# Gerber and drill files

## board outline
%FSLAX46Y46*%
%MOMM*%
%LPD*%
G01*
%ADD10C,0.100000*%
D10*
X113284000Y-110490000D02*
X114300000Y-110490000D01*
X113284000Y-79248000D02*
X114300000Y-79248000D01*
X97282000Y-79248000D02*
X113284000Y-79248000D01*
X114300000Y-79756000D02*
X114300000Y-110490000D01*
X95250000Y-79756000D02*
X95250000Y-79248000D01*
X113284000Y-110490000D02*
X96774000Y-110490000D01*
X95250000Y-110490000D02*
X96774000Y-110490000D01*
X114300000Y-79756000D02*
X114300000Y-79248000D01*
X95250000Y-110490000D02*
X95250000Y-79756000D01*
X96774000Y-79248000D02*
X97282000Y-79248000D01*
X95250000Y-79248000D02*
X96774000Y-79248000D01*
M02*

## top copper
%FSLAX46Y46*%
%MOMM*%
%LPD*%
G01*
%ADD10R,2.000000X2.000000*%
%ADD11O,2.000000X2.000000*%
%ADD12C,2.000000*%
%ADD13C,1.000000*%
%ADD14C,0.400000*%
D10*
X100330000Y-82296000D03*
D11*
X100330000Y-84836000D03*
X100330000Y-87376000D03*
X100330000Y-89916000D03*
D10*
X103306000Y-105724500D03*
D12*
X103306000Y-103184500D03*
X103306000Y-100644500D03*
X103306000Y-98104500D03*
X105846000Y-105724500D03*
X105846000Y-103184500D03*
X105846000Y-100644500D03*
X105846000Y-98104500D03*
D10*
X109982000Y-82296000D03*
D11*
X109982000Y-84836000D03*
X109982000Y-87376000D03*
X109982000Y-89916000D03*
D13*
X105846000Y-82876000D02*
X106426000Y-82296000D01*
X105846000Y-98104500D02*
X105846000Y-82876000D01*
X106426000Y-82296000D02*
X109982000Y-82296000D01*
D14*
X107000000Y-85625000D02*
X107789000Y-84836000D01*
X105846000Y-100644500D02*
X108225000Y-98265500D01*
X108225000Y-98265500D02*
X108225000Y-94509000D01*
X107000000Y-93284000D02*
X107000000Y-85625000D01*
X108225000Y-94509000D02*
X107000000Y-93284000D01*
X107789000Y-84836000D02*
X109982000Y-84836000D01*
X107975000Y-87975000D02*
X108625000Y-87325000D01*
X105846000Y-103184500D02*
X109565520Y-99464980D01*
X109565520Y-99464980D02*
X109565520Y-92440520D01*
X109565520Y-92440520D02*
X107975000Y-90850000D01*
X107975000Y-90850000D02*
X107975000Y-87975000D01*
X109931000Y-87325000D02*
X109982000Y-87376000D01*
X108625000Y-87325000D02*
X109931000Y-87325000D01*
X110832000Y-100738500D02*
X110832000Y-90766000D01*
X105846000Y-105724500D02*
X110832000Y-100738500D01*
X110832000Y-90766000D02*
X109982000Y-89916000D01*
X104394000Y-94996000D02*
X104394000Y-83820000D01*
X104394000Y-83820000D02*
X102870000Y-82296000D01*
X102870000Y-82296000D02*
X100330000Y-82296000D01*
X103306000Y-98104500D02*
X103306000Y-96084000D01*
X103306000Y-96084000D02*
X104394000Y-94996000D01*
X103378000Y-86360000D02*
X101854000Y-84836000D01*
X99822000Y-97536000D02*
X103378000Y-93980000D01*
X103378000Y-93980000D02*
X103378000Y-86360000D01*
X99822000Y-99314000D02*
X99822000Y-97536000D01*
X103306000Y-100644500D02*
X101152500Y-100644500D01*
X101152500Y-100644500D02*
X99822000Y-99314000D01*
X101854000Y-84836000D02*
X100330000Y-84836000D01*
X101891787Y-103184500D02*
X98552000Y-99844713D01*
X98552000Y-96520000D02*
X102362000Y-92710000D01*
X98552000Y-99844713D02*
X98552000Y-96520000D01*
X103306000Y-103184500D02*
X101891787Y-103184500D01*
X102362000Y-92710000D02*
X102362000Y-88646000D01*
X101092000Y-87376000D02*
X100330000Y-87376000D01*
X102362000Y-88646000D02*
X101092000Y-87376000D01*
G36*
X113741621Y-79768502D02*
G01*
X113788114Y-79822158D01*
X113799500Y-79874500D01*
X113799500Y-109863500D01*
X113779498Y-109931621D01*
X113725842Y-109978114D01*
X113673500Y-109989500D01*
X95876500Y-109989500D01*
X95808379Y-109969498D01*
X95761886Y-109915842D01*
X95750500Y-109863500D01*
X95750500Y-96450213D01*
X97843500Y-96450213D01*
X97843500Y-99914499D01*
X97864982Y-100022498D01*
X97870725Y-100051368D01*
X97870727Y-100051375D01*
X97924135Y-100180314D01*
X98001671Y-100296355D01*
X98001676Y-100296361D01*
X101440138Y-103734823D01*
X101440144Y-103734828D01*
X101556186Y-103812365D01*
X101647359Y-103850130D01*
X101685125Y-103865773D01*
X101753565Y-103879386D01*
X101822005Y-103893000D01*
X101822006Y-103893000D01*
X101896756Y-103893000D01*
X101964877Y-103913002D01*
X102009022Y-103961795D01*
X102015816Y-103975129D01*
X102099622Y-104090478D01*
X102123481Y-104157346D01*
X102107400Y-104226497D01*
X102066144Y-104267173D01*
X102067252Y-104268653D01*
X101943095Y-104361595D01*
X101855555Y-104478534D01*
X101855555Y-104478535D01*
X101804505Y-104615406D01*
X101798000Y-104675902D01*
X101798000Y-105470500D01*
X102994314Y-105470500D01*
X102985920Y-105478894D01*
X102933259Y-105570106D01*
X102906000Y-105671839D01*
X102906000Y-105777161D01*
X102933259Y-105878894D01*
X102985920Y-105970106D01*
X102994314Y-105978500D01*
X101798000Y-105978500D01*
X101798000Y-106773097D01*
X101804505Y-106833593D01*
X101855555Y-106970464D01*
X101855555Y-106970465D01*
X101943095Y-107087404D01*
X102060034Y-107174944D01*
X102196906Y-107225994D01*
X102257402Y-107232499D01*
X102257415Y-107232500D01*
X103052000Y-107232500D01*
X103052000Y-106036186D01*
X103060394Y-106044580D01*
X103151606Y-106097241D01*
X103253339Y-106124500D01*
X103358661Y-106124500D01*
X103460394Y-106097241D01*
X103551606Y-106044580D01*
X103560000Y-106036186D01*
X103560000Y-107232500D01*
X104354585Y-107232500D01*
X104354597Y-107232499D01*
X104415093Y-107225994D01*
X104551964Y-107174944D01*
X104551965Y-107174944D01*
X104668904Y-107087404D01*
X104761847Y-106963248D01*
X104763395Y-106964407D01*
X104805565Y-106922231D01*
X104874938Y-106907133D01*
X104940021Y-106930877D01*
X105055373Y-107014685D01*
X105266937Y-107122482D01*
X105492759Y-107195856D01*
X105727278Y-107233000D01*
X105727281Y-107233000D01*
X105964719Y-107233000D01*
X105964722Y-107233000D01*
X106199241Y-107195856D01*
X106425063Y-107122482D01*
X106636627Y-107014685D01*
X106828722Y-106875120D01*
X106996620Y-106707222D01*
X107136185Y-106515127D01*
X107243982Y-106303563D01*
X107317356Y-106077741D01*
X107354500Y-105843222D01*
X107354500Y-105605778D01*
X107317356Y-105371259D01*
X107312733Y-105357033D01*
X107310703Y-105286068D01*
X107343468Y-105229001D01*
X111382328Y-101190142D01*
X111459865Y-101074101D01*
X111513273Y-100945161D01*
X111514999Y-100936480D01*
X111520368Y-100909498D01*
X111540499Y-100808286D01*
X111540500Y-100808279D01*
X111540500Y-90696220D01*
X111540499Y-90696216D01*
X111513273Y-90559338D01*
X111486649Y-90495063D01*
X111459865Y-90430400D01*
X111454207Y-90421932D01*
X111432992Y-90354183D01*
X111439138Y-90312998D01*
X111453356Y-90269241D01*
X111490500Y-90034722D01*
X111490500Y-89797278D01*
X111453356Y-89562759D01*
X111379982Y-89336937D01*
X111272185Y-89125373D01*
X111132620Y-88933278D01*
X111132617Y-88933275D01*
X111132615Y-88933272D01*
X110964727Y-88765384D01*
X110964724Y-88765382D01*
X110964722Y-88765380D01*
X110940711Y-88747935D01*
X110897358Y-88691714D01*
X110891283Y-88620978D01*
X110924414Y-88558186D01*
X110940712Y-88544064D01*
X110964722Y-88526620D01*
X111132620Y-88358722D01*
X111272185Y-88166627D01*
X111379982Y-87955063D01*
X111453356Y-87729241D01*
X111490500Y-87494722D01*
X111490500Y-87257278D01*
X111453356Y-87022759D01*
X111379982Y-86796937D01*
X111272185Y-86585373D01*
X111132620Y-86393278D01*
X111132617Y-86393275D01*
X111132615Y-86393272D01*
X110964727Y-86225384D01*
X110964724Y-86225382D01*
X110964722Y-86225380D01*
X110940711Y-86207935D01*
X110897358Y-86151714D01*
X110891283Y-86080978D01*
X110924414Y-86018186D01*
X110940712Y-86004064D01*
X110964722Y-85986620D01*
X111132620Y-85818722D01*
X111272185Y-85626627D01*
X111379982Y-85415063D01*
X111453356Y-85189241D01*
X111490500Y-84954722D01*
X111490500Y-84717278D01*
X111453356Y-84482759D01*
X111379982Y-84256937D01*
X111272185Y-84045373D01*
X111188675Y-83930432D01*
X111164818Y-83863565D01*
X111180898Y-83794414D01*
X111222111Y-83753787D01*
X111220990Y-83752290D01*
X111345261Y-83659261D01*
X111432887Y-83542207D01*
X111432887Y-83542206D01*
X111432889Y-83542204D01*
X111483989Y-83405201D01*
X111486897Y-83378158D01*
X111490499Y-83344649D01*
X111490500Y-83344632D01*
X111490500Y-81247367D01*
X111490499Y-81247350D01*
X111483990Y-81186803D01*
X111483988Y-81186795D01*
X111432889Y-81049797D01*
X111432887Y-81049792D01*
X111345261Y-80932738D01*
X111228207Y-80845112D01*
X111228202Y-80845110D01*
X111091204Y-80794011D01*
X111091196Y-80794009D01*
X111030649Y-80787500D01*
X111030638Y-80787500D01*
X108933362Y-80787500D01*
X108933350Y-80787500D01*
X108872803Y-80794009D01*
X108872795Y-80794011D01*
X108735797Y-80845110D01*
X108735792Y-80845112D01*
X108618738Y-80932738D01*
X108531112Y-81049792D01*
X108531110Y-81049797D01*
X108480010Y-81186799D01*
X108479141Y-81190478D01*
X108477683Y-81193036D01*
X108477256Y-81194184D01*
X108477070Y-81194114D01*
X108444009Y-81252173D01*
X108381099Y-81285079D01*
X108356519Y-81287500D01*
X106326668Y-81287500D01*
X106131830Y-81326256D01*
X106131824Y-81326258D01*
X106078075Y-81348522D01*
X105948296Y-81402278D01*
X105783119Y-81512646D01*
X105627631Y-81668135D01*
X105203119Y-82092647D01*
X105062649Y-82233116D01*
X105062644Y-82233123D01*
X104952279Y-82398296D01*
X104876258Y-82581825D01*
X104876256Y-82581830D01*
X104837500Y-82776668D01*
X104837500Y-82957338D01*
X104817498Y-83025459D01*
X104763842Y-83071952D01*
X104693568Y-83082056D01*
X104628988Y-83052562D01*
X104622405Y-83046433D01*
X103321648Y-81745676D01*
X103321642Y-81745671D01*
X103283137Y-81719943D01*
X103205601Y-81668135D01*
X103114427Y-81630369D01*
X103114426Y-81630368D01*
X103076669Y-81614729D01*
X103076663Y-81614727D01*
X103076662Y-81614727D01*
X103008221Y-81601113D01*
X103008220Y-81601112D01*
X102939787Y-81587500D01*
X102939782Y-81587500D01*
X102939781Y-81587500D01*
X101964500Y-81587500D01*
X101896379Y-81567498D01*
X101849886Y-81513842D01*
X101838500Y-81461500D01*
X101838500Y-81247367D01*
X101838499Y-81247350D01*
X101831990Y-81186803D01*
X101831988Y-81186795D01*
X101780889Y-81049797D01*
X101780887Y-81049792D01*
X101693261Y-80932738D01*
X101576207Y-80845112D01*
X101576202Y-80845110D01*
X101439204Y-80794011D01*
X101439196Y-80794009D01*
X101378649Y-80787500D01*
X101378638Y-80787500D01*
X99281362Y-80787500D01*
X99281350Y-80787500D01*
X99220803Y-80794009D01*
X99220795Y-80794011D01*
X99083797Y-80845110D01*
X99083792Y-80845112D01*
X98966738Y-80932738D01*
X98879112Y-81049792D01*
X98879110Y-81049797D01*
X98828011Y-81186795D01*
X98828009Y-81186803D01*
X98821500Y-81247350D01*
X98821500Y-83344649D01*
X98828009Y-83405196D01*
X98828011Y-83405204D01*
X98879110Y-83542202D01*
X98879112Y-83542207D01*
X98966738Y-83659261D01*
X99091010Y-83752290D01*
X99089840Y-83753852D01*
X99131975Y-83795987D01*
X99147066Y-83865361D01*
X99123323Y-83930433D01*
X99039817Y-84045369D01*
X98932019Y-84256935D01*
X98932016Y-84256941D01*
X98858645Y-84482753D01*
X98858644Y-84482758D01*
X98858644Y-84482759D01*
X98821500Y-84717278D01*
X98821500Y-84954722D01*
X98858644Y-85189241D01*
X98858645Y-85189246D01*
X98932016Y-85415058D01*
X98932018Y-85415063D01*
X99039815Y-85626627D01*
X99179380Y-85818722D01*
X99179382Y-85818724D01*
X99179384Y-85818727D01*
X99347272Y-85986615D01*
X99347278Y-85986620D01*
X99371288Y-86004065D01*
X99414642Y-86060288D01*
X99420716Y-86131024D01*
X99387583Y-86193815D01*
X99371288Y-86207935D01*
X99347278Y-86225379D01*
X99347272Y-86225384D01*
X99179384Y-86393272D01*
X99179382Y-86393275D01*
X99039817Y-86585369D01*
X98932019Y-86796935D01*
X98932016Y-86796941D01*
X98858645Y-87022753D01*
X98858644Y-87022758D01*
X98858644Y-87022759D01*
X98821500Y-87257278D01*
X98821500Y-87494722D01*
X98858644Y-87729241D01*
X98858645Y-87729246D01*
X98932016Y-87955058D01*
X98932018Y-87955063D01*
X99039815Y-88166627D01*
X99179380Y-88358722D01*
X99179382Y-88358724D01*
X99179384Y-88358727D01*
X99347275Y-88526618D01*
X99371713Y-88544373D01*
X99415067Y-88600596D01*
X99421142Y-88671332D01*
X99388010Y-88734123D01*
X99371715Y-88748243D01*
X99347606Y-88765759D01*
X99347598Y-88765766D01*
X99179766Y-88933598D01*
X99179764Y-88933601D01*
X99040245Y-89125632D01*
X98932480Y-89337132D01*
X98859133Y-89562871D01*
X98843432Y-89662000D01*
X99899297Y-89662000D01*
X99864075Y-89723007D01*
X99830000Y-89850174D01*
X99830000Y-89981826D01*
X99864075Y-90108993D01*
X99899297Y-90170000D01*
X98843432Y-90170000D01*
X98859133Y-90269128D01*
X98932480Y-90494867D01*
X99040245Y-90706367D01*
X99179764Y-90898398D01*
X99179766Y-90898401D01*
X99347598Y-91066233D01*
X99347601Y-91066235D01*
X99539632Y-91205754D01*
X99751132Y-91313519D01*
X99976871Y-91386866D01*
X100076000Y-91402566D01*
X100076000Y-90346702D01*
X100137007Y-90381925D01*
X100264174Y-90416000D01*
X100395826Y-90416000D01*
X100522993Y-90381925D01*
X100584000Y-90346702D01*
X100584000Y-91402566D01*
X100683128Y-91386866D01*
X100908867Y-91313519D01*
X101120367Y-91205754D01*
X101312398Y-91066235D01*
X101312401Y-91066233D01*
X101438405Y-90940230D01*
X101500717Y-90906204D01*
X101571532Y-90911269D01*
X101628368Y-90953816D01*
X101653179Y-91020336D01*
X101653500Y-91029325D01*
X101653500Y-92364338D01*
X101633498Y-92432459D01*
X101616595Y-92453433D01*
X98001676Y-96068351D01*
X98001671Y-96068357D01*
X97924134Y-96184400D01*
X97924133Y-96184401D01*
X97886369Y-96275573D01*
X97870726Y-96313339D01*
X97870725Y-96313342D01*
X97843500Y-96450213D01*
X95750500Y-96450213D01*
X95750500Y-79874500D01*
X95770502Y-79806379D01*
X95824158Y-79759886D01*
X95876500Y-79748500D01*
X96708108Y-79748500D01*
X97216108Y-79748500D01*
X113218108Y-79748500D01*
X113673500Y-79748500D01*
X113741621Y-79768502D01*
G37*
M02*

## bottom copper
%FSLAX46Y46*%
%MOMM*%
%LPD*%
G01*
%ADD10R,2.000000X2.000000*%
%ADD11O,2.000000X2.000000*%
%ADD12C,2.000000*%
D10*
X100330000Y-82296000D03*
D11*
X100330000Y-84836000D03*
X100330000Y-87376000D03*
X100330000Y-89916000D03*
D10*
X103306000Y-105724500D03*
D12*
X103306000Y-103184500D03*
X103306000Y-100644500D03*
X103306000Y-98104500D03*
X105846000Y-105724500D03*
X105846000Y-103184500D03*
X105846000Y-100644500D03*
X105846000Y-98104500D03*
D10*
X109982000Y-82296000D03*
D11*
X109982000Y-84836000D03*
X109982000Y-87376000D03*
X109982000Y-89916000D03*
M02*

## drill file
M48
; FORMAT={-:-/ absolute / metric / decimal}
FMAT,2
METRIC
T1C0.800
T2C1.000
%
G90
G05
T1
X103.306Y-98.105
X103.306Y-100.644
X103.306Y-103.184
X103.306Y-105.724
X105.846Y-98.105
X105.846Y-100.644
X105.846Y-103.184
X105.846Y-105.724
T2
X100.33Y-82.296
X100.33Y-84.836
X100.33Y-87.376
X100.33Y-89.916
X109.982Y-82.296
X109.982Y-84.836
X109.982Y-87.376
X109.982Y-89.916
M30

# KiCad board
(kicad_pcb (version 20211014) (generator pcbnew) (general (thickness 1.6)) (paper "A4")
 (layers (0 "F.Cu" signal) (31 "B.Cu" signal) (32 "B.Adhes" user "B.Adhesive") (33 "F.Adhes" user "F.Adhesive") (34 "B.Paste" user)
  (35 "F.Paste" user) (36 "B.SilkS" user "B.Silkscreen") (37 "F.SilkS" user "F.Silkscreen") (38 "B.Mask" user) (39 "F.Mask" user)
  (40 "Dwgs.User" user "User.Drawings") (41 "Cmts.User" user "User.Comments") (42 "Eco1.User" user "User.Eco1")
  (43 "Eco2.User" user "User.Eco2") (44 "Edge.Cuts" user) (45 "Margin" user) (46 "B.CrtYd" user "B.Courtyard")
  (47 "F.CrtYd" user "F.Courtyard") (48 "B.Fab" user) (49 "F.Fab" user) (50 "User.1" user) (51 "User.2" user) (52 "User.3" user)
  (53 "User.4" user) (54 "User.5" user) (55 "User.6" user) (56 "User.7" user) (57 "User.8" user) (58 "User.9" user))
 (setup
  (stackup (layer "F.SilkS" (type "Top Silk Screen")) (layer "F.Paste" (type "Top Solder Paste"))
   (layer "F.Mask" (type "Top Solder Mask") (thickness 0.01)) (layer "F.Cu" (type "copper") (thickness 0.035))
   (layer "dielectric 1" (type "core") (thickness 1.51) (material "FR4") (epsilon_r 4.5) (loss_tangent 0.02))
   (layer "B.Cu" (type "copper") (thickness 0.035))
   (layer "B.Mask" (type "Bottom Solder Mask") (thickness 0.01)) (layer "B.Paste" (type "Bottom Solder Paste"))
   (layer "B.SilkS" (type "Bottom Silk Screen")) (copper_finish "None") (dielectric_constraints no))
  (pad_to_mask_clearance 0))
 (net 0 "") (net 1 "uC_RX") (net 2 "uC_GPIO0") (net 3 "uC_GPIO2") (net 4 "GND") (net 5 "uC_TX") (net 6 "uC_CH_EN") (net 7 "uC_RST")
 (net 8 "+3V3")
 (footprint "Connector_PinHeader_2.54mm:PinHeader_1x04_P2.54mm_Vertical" (layer "F.Cu") (at 100.33 82.296)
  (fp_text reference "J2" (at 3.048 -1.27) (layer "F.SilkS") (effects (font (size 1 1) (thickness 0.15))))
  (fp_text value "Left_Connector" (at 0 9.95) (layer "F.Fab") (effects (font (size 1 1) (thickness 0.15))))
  (pad "1" thru_hole rect (at 0 0) (size 2 2) (drill 1) (layers *.Cu *.Mask) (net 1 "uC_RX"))
  (pad "2" thru_hole oval (at 0 2.54) (size 2 2) (drill 1) (layers *.Cu *.Mask) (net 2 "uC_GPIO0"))
  (pad "3" thru_hole oval (at 0 5.08) (size 2 2) (drill 1) (layers *.Cu *.Mask) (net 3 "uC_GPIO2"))
  (pad "4" thru_hole oval (at 0 7.62) (size 2 2) (drill 1) (layers *.Cu *.Mask) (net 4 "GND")))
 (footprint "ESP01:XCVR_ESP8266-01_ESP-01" (layer "F.Cu") (at 94.996 101.9145 90)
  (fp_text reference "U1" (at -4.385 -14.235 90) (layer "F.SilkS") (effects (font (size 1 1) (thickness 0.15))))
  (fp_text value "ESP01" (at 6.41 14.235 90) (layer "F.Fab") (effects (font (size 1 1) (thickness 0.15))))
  (pad "1" thru_hole rect (at -3.81 8.31 90) (size 2 2) (drill 0.8) (layers *.Cu *.Mask) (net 4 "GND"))
  (pad "2" thru_hole circle (at -1.27 8.31 90) (size 2 2) (drill 0.8) (layers *.Cu *.Mask) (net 3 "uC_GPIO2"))
  (pad "3" thru_hole circle (at 1.27 8.31 90) (size 2 2) (drill 0.8) (layers *.Cu *.Mask) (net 2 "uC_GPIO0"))
  (pad "4" thru_hole circle (at 3.81 8.31 90) (size 2 2) (drill 0.8) (layers *.Cu *.Mask) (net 1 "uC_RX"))
  (pad "5" thru_hole circle (at -3.81 10.85 90) (size 2 2) (drill 0.8) (layers *.Cu *.Mask) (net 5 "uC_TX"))
  (pad "6" thru_hole circle (at -1.27 10.85 90) (size 2 2) (drill 0.8) (layers *.Cu *.Mask) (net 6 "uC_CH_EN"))
  (pad "7" thru_hole circle (at 1.27 10.85 90) (size 2 2) (drill 0.8) (layers *.Cu *.Mask) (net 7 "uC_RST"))
  (pad "8" thru_hole circle (at 3.81 10.85 90) (size 2 2) (drill 0.8) (layers *.Cu *.Mask) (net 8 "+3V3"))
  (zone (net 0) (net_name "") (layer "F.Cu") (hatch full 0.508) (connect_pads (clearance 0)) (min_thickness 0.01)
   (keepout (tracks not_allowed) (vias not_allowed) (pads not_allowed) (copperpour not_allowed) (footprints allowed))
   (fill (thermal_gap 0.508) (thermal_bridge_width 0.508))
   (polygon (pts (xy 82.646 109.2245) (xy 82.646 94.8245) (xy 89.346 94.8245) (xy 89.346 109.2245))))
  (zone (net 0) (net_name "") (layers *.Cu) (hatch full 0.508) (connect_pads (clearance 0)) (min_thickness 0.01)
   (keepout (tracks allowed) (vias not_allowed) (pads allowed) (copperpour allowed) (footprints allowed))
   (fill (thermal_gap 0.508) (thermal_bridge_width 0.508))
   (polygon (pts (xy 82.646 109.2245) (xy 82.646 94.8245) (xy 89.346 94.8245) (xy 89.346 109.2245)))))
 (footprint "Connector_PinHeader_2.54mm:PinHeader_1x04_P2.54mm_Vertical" (layer "F.Cu") (at 109.982 82.296)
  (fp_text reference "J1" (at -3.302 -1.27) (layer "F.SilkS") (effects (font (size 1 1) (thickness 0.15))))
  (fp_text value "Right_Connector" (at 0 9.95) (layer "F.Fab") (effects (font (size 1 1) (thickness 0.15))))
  (pad "1" thru_hole rect (at 0 0) (size 2 2) (drill 1) (layers *.Cu *.Mask) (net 8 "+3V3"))
  (pad "2" thru_hole oval (at 0 2.54) (size 2 2) (drill 1) (layers *.Cu *.Mask) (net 7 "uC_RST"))
  (pad "3" thru_hole oval (at 0 5.08) (size 2 2) (drill 1) (layers *.Cu *.Mask) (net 6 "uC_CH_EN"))
  (pad "4" thru_hole oval (at 0 7.62) (size 2 2) (drill 1) (layers *.Cu *.Mask) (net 5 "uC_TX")))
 (gr_line (start 113.284 110.49) (end 114.3 110.49) (layer "Edge.Cuts") (width 0.1))
 (gr_line (start 113.284 79.248) (end 114.3 79.248) (layer "Edge.Cuts") (width 0.1))
 (gr_line (start 97.282 79.248) (end 113.284 79.248) (layer "Edge.Cuts") (width 0.1))
 (gr_line (start 114.3 79.756) (end 114.3 110.49) (layer "Edge.Cuts") (width 0.1))
 (gr_line (start 95.25 79.756) (end 95.25 79.248) (layer "Edge.Cuts") (width 0.1))
 (gr_line (start 113.284 110.49) (end 96.774 110.49) (layer "Edge.Cuts") (width 0.1))
 (gr_line (start 95.25 110.49) (end 96.774 110.49) (layer "Edge.Cuts") (width 0.1))
 (gr_line (start 114.3 79.756) (end 114.3 79.248) (layer "Edge.Cuts") (width 0.1))
 (gr_line (start 95.25 110.49) (end 95.25 79.756) (layer "Edge.Cuts") (width 0.1))
 (gr_line (start 96.774 79.248) (end 97.282 79.248) (layer "Edge.Cuts") (width 0.1))
 (gr_line (start 95.25 79.248) (end 96.774 79.248) (layer "Edge.Cuts") (width 0.1))
 (segment (start 105.846 82.876) (end 106.426 82.296) (width 1) (layer "F.Cu") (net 8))
 (segment (start 105.846 98.1045) (end 105.846 82.876) (width 1) (layer "F.Cu") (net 8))
 (segment (start 106.426 82.296) (end 109.982 82.296) (width 1) (layer "F.Cu") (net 8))
 (segment (start 107 85.625) (end 107.789 84.836) (width 0.4) (layer "F.Cu") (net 7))
 (segment (start 105.846 100.6445) (end 108.225 98.2655) (width 0.4) (layer "F.Cu") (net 7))
 (segment (start 108.225 98.2655) (end 108.225 94.509) (width 0.4) (layer "F.Cu") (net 7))
 (segment (start 107 93.284) (end 107 85.625) (width 0.4) (layer "F.Cu") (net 7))
 (segment (start 108.225 94.509) (end 107 93.284) (width 0.4) (layer "F.Cu") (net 7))
 (segment (start 107.789 84.836) (end 109.982 84.836) (width 0.4) (layer "F.Cu") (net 7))
 (segment (start 107.975 87.975) (end 108.625 87.325) (width 0.4) (layer "F.Cu") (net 6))
 (segment (start 105.846 103.1845) (end 109.56552 99.46498) (width 0.4) (layer "F.Cu") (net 6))
 (segment (start 109.56552 99.46498) (end 109.56552 92.44052) (width 0.4) (layer "F.Cu") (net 6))
 (segment (start 109.56552 92.44052) (end 107.975 90.85) (width 0.4) (layer "F.Cu") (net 6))
 (segment (start 107.975 90.85) (end 107.975 87.975) (width 0.4) (layer "F.Cu") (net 6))
 (segment (start 109.931 87.325) (end 109.982 87.376) (width 0.4) (layer "F.Cu") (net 6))
 (segment (start 108.625 87.325) (end 109.931 87.325) (width 0.4) (layer "F.Cu") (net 6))
 (segment (start 110.832 100.7385) (end 110.832 90.766) (width 0.4) (layer "F.Cu") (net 5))
 (segment (start 105.846 105.7245) (end 110.832 100.7385) (width 0.4) (layer "F.Cu") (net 5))
 (segment (start 110.832 90.766) (end 109.982 89.916) (width 0.4) (layer "F.Cu") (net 5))
 (segment (start 104.394 94.996) (end 104.394 83.82) (width 0.4) (layer "F.Cu") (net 1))
 (segment (start 104.394 83.82) (end 102.87 82.296) (width 0.4) (layer "F.Cu") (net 1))
 (segment (start 102.87 82.296) (end 100.33 82.296) (width 0.4) (layer "F.Cu") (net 1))
 (segment (start 103.306 98.1045) (end 103.306 96.084) (width 0.4) (layer "F.Cu") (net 1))
 (segment (start 103.306 96.084) (end 104.394 94.996) (width 0.4) (layer "F.Cu") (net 1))
 (segment (start 103.378 86.36) (end 101.854 84.836) (width 0.4) (layer "F.Cu") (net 2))
 (segment (start 99.822 97.536) (end 103.378 93.98) (width 0.4) (layer "F.Cu") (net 2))
 (segment (start 103.378 93.98) (end 103.378 86.36) (width 0.4) (layer "F.Cu") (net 2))
 (segment (start 99.822 99.314) (end 99.822 97.536) (width 0.4) (layer "F.Cu") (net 2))
 (segment (start 103.306 100.6445) (end 101.1525 100.6445) (width 0.4) (layer "F.Cu") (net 2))
 (segment (start 101.1525 100.6445) (end 99.822 99.314) (width 0.4) (layer "F.Cu") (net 2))
 (segment (start 101.854 84.836) (end 100.33 84.836) (width 0.4) (layer "F.Cu") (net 2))
 (segment (start 101.891787 103.1845) (end 98.552 99.844713) (width 0.4) (layer "F.Cu") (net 3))
 (segment (start 98.552 96.52) (end 102.362 92.71) (width 0.4) (layer "F.Cu") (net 3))
 (segment (start 98.552 99.844713) (end 98.552 96.52) (width 0.4) (layer "F.Cu") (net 3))
 (segment (start 103.306 103.1845) (end 101.891787 103.1845) (width 0.4) (layer "F.Cu") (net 3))
 (segment (start 102.362 92.71) (end 102.362 88.646) (width 0.4) (layer "F.Cu") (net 3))
 (segment (start 101.092 87.376) (end 100.33 87.376) (width 0.4) (layer "F.Cu") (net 3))
 (segment (start 102.362 88.646) (end 101.092 87.376) (width 0.4) (layer "F.Cu") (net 3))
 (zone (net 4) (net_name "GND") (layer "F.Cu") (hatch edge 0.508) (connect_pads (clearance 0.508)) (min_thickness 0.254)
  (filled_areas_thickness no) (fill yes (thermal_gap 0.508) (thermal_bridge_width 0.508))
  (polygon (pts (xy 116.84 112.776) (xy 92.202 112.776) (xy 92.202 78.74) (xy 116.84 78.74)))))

